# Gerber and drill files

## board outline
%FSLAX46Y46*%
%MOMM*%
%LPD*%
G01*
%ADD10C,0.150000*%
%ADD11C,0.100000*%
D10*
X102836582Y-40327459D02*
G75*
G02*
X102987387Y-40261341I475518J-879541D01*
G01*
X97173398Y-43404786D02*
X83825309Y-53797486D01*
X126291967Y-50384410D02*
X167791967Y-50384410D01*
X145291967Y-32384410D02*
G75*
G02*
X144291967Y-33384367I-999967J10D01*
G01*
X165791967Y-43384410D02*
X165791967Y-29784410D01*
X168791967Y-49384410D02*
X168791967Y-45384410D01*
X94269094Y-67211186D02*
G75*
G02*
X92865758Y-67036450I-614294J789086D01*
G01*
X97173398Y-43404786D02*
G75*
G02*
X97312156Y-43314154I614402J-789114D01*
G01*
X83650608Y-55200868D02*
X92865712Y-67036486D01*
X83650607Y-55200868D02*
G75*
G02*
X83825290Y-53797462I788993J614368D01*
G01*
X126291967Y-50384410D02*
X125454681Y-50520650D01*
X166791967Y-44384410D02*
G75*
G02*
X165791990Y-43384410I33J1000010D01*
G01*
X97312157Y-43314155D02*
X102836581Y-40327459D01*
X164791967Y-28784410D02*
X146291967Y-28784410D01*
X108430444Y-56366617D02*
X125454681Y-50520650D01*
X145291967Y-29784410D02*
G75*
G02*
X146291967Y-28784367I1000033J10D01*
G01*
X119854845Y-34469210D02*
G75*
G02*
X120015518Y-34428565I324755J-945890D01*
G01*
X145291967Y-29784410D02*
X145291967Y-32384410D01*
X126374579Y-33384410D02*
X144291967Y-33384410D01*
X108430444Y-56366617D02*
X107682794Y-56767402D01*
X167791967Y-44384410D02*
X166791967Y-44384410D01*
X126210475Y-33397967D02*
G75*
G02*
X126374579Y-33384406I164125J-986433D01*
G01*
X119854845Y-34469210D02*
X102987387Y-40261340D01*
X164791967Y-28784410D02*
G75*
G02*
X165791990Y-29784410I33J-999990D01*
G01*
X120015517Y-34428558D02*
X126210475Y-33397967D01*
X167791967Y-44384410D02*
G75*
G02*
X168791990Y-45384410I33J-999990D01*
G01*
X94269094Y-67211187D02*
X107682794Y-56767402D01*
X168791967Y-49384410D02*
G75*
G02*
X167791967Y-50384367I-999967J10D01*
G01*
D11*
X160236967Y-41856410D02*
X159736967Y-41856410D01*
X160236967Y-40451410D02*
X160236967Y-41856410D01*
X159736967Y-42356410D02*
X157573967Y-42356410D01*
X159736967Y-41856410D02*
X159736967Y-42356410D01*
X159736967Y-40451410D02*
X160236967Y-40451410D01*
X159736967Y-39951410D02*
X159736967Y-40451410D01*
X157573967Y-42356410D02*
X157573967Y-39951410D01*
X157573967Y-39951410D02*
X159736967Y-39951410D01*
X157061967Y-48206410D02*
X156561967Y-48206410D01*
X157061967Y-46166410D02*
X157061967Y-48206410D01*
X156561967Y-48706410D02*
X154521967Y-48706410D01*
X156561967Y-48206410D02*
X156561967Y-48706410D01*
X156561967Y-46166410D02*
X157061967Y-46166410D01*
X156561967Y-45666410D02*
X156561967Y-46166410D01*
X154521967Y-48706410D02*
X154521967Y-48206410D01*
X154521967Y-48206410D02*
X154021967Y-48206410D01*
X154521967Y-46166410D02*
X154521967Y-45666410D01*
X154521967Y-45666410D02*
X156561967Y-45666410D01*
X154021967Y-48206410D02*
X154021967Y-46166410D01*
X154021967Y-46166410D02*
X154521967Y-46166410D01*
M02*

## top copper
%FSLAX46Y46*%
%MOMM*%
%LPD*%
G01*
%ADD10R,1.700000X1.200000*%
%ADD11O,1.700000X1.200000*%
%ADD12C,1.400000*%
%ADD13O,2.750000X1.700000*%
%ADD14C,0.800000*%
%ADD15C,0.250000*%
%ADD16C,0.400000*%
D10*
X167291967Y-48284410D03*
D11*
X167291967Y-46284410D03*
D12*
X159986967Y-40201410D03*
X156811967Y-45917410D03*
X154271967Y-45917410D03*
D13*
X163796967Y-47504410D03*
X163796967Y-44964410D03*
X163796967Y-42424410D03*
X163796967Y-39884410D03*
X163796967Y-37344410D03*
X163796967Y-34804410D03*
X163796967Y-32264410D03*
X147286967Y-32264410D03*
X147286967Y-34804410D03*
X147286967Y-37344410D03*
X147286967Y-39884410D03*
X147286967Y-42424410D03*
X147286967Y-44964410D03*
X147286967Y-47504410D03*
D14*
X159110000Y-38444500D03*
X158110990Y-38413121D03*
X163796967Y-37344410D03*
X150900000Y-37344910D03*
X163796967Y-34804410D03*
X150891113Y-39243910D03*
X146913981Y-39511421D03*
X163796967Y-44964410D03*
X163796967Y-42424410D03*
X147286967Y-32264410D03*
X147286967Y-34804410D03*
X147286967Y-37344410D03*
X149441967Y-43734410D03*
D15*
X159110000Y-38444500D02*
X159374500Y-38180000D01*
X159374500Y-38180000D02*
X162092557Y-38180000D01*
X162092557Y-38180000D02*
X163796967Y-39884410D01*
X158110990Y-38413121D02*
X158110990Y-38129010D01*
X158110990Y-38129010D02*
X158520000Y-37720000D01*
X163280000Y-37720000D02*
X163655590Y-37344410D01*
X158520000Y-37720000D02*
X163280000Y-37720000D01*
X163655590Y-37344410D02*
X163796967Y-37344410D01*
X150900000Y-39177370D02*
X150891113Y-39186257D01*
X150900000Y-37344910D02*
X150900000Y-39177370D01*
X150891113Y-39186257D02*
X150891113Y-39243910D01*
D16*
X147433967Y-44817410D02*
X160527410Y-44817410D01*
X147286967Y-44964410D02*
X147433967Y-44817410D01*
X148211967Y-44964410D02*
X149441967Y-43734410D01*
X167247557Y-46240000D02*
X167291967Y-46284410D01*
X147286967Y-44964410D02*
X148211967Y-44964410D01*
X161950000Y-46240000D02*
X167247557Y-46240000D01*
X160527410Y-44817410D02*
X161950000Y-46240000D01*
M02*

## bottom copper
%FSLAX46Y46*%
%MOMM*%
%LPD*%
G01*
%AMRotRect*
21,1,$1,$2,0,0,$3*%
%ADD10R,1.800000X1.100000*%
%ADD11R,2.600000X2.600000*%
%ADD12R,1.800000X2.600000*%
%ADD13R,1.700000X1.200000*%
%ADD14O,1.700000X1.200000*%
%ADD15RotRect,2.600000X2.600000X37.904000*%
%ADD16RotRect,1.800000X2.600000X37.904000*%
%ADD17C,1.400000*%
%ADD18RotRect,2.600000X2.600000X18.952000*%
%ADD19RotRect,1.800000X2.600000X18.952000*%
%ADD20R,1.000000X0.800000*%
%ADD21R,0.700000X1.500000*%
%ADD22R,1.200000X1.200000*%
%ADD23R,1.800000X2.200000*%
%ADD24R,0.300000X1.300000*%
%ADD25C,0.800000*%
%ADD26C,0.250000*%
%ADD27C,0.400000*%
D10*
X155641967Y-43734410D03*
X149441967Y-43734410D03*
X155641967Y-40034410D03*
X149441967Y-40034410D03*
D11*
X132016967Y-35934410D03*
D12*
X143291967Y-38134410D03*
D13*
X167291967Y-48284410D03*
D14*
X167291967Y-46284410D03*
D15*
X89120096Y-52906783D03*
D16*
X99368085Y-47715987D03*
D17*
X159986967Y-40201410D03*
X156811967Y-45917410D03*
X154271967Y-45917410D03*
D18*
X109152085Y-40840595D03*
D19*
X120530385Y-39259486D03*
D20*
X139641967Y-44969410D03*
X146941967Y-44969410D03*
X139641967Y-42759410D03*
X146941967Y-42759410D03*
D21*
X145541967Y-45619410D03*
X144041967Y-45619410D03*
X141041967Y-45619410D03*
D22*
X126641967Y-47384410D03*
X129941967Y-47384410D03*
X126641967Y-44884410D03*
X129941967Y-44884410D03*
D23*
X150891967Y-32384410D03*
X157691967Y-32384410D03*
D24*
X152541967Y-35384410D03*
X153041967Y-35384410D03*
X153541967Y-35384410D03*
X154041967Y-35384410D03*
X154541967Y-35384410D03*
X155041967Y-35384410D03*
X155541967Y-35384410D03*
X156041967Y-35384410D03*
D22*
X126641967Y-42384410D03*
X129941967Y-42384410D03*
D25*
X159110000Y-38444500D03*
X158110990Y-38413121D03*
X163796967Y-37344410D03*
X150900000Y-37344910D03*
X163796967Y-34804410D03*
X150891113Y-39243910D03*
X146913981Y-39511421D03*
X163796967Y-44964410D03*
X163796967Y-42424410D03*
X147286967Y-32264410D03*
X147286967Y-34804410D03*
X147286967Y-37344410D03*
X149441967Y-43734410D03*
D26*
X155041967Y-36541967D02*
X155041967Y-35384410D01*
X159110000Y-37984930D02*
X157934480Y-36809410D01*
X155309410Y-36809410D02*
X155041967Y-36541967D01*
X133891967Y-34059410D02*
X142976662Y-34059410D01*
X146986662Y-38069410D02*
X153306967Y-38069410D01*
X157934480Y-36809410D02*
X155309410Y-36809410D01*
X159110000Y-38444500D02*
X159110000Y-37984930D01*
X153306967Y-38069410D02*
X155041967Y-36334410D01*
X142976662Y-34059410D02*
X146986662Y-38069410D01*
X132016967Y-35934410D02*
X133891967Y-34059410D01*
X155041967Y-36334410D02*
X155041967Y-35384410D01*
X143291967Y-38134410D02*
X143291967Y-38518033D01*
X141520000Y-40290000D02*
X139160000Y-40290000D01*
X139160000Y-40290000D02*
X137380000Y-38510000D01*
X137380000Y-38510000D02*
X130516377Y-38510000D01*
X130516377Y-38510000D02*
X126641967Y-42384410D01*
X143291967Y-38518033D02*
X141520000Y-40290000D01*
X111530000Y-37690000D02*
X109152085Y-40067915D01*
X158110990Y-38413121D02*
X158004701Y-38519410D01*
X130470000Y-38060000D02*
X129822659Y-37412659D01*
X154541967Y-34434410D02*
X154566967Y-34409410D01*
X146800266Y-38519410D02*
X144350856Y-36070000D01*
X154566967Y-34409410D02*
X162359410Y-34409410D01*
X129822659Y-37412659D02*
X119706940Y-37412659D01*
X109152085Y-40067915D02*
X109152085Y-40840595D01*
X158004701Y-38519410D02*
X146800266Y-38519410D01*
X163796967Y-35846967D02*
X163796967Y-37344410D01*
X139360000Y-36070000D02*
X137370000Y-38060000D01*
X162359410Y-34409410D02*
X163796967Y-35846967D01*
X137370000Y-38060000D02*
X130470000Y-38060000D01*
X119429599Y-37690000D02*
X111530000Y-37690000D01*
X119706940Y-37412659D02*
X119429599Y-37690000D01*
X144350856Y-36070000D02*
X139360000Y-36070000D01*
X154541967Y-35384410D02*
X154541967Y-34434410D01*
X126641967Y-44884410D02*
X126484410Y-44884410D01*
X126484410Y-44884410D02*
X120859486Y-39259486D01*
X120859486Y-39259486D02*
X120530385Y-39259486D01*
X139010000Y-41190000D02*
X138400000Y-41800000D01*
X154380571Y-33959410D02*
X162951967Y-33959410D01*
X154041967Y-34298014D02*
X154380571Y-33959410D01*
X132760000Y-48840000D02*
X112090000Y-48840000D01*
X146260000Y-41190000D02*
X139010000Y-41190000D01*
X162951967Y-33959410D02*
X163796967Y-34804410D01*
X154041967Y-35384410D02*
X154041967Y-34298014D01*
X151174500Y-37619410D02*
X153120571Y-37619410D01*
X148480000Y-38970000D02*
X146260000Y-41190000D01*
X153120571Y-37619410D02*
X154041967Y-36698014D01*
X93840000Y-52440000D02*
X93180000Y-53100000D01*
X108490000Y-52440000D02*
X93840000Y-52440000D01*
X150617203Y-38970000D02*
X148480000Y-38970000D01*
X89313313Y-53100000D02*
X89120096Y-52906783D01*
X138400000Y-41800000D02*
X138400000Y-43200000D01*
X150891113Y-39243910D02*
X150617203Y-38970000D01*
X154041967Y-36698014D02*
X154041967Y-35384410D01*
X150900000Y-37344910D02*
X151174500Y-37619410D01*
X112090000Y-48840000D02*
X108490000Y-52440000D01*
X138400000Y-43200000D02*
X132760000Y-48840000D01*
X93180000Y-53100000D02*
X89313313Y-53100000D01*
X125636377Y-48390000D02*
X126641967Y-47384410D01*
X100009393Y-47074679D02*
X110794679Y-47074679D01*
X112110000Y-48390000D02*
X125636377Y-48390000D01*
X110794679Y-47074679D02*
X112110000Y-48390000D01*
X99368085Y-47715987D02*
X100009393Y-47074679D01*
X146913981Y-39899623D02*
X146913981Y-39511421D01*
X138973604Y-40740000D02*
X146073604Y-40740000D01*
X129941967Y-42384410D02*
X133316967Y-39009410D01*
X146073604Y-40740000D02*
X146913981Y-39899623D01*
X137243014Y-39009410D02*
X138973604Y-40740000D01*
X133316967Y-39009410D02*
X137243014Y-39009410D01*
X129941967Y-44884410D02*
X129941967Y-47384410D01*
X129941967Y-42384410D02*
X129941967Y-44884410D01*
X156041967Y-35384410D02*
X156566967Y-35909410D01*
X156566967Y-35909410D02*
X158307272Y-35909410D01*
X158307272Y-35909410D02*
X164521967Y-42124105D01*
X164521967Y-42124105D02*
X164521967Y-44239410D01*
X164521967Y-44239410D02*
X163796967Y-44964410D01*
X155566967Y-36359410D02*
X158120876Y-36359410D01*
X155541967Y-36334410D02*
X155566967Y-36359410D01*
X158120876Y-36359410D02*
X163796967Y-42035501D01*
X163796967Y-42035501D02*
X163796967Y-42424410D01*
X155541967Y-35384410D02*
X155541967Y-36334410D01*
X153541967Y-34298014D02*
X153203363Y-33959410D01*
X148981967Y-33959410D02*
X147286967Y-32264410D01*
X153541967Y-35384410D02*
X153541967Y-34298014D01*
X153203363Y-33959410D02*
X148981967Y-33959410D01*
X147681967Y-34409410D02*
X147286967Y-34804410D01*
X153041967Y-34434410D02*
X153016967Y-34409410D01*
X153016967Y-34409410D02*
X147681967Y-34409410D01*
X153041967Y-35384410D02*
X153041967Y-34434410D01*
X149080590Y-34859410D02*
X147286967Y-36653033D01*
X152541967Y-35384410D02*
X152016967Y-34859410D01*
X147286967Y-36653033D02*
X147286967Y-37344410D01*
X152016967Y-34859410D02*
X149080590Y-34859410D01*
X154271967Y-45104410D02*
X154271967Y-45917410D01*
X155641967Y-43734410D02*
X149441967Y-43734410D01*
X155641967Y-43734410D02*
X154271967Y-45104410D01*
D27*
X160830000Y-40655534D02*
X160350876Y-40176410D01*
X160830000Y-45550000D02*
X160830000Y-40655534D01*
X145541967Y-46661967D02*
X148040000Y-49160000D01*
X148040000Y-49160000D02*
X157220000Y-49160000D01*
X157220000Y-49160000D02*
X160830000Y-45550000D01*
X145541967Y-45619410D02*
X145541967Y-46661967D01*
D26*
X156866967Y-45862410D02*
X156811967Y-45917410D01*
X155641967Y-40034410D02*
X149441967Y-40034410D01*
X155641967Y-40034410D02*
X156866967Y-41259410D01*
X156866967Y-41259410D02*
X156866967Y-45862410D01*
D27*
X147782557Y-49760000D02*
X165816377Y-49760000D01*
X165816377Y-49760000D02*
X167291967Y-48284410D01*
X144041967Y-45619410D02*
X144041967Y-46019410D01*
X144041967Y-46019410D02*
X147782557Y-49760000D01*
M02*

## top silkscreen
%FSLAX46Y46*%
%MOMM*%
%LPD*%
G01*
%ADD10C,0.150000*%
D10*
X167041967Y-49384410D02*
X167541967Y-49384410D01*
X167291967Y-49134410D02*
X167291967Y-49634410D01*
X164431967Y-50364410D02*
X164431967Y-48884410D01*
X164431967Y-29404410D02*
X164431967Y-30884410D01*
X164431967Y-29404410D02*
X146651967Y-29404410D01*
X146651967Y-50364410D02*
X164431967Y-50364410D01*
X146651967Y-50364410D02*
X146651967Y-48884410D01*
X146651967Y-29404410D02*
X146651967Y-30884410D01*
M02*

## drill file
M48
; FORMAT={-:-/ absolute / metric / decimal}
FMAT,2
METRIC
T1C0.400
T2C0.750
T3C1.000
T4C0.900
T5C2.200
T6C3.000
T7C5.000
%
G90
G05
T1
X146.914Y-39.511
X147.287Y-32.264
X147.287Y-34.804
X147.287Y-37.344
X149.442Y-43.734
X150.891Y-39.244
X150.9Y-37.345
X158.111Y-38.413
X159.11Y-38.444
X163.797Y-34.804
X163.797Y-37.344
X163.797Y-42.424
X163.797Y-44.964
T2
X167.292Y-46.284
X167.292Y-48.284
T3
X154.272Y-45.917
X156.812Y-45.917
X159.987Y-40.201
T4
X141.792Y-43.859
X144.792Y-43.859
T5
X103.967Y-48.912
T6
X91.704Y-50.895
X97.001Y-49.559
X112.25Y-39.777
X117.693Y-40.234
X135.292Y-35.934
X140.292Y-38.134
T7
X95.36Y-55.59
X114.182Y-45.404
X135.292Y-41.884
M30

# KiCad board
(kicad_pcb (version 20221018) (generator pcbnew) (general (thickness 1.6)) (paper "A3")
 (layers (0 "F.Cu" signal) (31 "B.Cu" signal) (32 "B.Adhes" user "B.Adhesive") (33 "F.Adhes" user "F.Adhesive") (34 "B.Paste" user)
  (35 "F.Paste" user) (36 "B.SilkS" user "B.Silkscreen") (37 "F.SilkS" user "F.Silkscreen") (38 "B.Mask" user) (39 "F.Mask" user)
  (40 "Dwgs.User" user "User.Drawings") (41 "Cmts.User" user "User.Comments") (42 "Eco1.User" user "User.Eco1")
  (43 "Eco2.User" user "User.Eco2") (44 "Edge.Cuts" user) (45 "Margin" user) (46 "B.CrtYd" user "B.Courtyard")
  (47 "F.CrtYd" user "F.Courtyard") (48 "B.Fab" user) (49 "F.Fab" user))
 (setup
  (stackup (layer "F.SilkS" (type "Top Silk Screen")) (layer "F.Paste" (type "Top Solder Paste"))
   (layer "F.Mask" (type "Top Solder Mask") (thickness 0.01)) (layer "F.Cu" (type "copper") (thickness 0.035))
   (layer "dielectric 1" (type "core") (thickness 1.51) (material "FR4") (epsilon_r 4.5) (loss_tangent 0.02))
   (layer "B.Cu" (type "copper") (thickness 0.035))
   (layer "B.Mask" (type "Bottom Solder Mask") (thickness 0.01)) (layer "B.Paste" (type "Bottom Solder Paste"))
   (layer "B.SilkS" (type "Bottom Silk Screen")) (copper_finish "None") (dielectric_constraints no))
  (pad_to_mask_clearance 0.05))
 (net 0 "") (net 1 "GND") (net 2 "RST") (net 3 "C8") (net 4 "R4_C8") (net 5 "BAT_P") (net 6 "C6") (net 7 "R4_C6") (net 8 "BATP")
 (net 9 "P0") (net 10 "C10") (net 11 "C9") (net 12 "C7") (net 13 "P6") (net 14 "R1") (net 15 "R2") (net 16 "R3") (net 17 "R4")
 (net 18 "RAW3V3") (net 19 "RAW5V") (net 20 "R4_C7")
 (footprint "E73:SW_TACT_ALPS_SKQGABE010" (layer "F.Cu") (at 152.541967 41.88441 180)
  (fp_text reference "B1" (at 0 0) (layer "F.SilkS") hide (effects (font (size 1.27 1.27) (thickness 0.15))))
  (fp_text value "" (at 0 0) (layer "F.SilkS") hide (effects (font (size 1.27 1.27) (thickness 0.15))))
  (pad "1" smd rect (at -3.1 -1.85 180) (size 1.8 1.1) (layers "B.Cu" "B.Paste" "B.Mask") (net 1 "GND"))
  (pad "1" smd rect (at 3.1 -1.85 180) (size 1.8 1.1) (layers "B.Cu" "B.Paste" "B.Mask") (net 1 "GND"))
  (pad "2" smd rect (at -3.1 1.85 180) (size 1.8 1.1) (layers "B.Cu" "B.Paste" "B.Mask") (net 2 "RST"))
  (pad "2" smd rect (at 3.1 1.85 180) (size 1.8 1.1) (layers "B.Cu" "B.Paste" "B.Mask") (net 2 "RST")))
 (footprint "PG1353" (layer "F.Cu") (at 135.291967 41.88441)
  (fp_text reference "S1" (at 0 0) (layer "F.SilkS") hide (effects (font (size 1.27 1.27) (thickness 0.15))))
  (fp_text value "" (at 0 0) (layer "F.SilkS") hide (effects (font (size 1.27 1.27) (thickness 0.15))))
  (pad "" np_thru_hole circle (at 0 -5.95) (size 3 3) (drill 3) (layers "*.Cu" "*.Mask"))
  (pad "" np_thru_hole circle (at 0 0) (size 5 5) (drill 5) (layers "*.Cu" "*.Mask"))
  (pad "" np_thru_hole circle (at 5 -3.75) (size 3 3) (drill 3) (layers "*.Cu" "*.Mask"))
  (pad "1" smd rect (at -3.275 -5.95) (size 2.6 2.6) (layers "B.Cu" "B.Paste" "B.Mask") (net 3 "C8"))
  (pad "2" smd rect (at 8 -3.75) (size 1.8 2.6) (layers "B.Cu" "B.Paste" "B.Mask") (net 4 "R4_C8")))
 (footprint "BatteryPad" (layer "F.Cu") (at 167.291967 47.28441 90)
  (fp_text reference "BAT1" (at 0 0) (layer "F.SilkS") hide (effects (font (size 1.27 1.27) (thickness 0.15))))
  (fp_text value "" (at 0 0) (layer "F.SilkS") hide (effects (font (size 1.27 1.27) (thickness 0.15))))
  (fp_line (start -2.1 -0.25) (end -2.1 0.25) (stroke (width 0.15) (type solid)) (layer "F.SilkS"))
  (fp_line (start -1.85 0) (end -2.35 0) (stroke (width 0.15) (type solid)) (layer "F.SilkS"))
  (pad "1" thru_hole rect (at -1 0 90) (size 1.2 1.7) (drill 0.75) (layers "*.Cu" "*.Mask") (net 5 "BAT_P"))
  (pad "2" thru_hole oval (at 1 0 90) (size 1.2 1.7) (drill 0.75) (layers "*.Cu" "*.Mask") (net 1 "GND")))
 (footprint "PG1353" (layer "F.Cu") (at 95.359531 55.589614 37.904)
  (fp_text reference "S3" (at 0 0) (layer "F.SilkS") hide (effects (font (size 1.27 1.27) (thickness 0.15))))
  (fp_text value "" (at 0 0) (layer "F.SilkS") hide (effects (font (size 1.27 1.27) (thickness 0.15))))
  (pad "" np_thru_hole circle (at 0 -5.95) (size 3 3) (drill 3) (layers "*.Cu" "*.Mask"))
  (pad "" np_thru_hole circle (at 0 0) (size 5 5) (drill 5) (layers "*.Cu" "*.Mask"))
  (pad "" np_thru_hole circle (at 5 -3.75) (size 3 3) (drill 3) (layers "*.Cu" "*.Mask"))
  (pad "1" smd rect (at -3.275 -5.95 37.904) (size 2.6 2.6) (layers "B.Cu" "B.Paste" "B.Mask") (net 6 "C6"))
  (pad "2" smd rect (at 8 -3.75 37.904) (size 1.8 2.6) (layers "B.Cu" "B.Paste" "B.Mask") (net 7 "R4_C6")))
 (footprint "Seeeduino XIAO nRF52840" (layer "F.Cu") (at 155.541967 39.88441 180)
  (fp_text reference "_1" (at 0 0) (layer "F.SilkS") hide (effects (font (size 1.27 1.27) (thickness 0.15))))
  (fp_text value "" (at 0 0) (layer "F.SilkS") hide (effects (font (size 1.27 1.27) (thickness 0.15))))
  (fp_line (start -8.89 -10.48) (end -8.89 -9) (stroke (width 0.15) (type solid)) (layer "F.SilkS"))
  (fp_line (start -8.89 10.48) (end -8.89 9) (stroke (width 0.15) (type solid)) (layer "F.SilkS"))
  (fp_line (start -8.89 10.48) (end 8.89 10.48) (stroke (width 0.15) (type solid)) (layer "F.SilkS"))
  (fp_line (start 8.89 -10.48) (end -8.89 -10.48) (stroke (width 0.15) (type solid)) (layer "F.SilkS"))
  (fp_line (start 8.89 -10.48) (end 8.89 -9) (stroke (width 0.15) (type solid)) (layer "F.SilkS"))
  (fp_line (start 8.89 10.48) (end 8.89 9) (stroke (width 0.15) (type solid)) (layer "F.SilkS"))
  (fp_line (start -4.695 -1.972) (end -4.195 -1.972) (stroke (width 0.1) (type solid)) (layer "Edge.Cuts"))
  (fp_line (start -4.695 -0.567) (end -4.695 -1.972) (stroke (width 0.1) (type solid)) (layer "Edge.Cuts"))
  (fp_line (start -4.195 -2.472) (end -2.032 -2.472) (stroke (width 0.1) (type solid)) (layer "Edge.Cuts"))
  (fp_line (start -4.195 -1.972) (end -4.195 -2.472) (stroke (width 0.1) (type solid)) (layer "Edge.Cuts"))
  (fp_line (start -4.195 -0.567) (end -4.695 -0.567) (stroke (width 0.1) (type solid)) (layer "Edge.Cuts"))
  (fp_line (start -4.195 -0.067) (end -4.195 -0.567) (stroke (width 0.1) (type solid)) (layer "Edge.Cuts"))
  (fp_line (start -2.032 -2.472) (end -2.032 -0.067) (stroke (width 0.1) (type solid)) (layer "Edge.Cuts"))
  (fp_line (start -2.032 -0.067) (end -4.195 -0.067) (stroke (width 0.1) (type solid)) (layer "Edge.Cuts"))
  (fp_line (start -1.52 -8.322) (end -1.02 -8.322) (stroke (width 0.1) (type solid)) (layer "Edge.Cuts"))
  (fp_line (start -1.52 -6.282) (end -1.52 -8.322) (stroke (width 0.1) (type solid)) (layer "Edge.Cuts"))
  (fp_line (start -1.02 -8.822) (end 1.02 -8.822) (stroke (width 0.1) (type solid)) (layer "Edge.Cuts"))
  (fp_line (start -1.02 -8.322) (end -1.02 -8.822) (stroke (width 0.1) (type solid)) (layer "Edge.Cuts"))
  (fp_line (start -1.02 -6.282) (end -1.52 -6.282) (stroke (width 0.1) (type solid)) (layer "Edge.Cuts"))
  (fp_line (start -1.02 -5.782) (end -1.02 -6.282) (stroke (width 0.1) (type solid)) (layer "Edge.Cuts"))
  (fp_line (start 1.02 -8.822) (end 1.02 -8.322) (stroke (width 0.1) (type solid)) (layer "Edge.Cuts"))
  (fp_line (start 1.02 -8.322) (end 1.52 -8.322) (stroke (width 0.1) (type solid)) (layer "Edge.Cuts"))
  (fp_line (start 1.02 -6.282) (end 1.02 -5.782) (stroke (width 0.1) (type solid)) (layer "Edge.Cuts"))
  (fp_line (start 1.02 -5.782) (end -1.02 -5.782) (stroke (width 0.1) (type solid)) (layer "Edge.Cuts"))
  (fp_line (start 1.52 -8.322) (end 1.52 -6.282) (stroke (width 0.1) (type solid)) (layer "Edge.Cuts"))
  (fp_line (start 1.52 -6.282) (end 1.02 -6.282) (stroke (width 0.1) (type solid)) (layer "Edge.Cuts"))
  (pad "" thru_hole circle (at -4.445 -0.317) (size 1.4 1.4) (drill 1) (layers "*.Cu" "*.Mask") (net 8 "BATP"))
  (pad "" thru_hole circle (at -1.27 -6.033) (size 1.4 1.4) (drill 1) (layers "*.Cu" "*.Mask") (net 2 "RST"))
  (pad "" thru_hole circle (at 1.27 -6.033) (size 1.4 1.4) (drill 1) (layers "*.Cu" "*.Mask") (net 1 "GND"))
  (pad "1" smd oval (at -8.255 -7.62 180) (size 2.75 1.7) (layers "F.Cu" "F.Paste" "F.Mask") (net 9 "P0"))
  (pad "2" smd oval (at -8.255 -5.08 180) (size 2.75 1.7) (layers "F.Cu" "F.Paste" "F.Mask") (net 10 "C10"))
  (pad "3" smd oval (at -8.255 -2.54 180) (size 2.75 1.7) (layers "F.Cu" "F.Paste" "F.Mask") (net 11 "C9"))
  (pad "4" smd oval (at -8.255 0 180) (size 2.75 1.7) (layers "F.Cu" "F.Paste" "F.Mask") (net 3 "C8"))
  (pad "5" smd oval (at -8.255 2.54 180) (size 2.75 1.7) (layers "F.Cu" "F.Paste" "F.Mask") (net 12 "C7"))
  (pad "6" smd oval (at -8.255 5.08 180) (size 2.75 1.7) (layers "F.Cu" "F.Paste" "F.Mask") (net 6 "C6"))
  (pad "7" smd oval (at -8.255 7.62 180) (size 2.75 1.7) (layers "F.Cu" "F.Paste" "F.Mask") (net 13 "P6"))
  (pad "8" smd oval (at 8.255 7.62 180) (size 2.75 1.7) (layers "F.Cu" "F.Paste" "F.Mask") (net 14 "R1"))
  (pad "9" smd oval (at 8.255 5.08 180) (size 2.75 1.7) (layers "F.Cu" "F.Paste" "F.Mask") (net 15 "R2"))
  (pad "10" smd oval (at 8.255 2.54 180) (size 2.75 1.7) (layers "F.Cu" "F.Paste" "F.Mask") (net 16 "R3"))
  (pad "11" smd oval (at 8.255 0 180) (size 2.75 1.7) (layers "F.Cu" "F.Paste" "F.Mask") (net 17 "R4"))
  (pad "12" smd oval (at 8.255 -2.54 180) (size 2.75 1.7) (layers "F.Cu" "F.Paste" "F.Mask") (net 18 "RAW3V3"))
  (pad "13" smd oval (at 8.255 -5.08 180) (size 2.75 1.7) (layers "F.Cu" "F.Paste" "F.Mask") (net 1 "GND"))
  (pad "14" smd oval (at 8.255 -7.62 180) (size 2.75 1.7) (layers "F.Cu" "F.Paste" "F.Mask") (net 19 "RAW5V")))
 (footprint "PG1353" (layer "F.Cu") (at 114.181967 45.40441 18.952)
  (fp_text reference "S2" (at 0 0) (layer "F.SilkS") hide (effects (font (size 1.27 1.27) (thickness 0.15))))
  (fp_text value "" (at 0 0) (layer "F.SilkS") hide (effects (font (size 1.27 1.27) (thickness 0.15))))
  (pad "" np_thru_hole circle (at 0 -5.95) (size 3 3) (drill 3) (layers "*.Cu" "*.Mask"))
  (pad "" np_thru_hole circle (at 0 0) (size 5 5) (drill 5) (layers "*.Cu" "*.Mask"))
  (pad "" np_thru_hole circle (at 5 -3.75) (size 3 3) (drill 3) (layers "*.Cu" "*.Mask"))
  (pad "1" smd rect (at -3.275 -5.95 18.952) (size 2.6 2.6) (layers "B.Cu" "B.Paste" "B.Mask") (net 12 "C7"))
  (pad "2" smd rect (at 8 -3.75 18.952) (size 1.8 2.6) (layers "B.Cu" "B.Paste" "B.Mask") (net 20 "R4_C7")))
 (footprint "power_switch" (layer "F.Cu") (at 143.291967 43.88441 90)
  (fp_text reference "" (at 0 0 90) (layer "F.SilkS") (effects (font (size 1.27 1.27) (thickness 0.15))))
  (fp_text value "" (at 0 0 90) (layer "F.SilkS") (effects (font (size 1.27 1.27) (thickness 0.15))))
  (pad "" smd rect (at -1.085 -3.65) (size 1 0.8) (layers "B.Cu" "B.Paste" "B.Mask"))
  (pad "" smd rect (at -1.085 3.65) (size 1 0.8) (layers "B.Cu" "B.Paste" "B.Mask"))
  (pad "" np_thru_hole circle (at 0.025 -1.5 180) (size 0.9 0.9) (drill 0.9) (layers "*.Cu" "*.Mask"))
  (pad "" np_thru_hole circle (at 0.025 1.5 180) (size 0.9 0.9) (drill 0.9) (layers "*.Cu" "*.Mask"))
  (pad "" smd rect (at 1.125 -3.65) (size 1 0.8) (layers "B.Cu" "B.Paste" "B.Mask"))
  (pad "" smd rect (at 1.125 3.65) (size 1 0.8) (layers "B.Cu" "B.Paste" "B.Mask"))
  (pad "4" smd rect (at -1.735 2.25) (size 0.7 1.5) (layers "B.Cu" "B.Paste" "B.Mask") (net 8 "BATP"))
  (pad "5" smd rect (at -1.735 0.75) (size 0.7 1.5) (layers "B.Cu" "B.Paste" "B.Mask") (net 5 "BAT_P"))
  (pad "6" smd rect (at -1.735 -2.25) (size 0.7 1.5) (layers "B.Cu" "B.Paste" "B.Mask")))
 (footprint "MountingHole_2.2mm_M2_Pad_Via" (layer "F.Cu") (at 103.967424 48.91199 18.952)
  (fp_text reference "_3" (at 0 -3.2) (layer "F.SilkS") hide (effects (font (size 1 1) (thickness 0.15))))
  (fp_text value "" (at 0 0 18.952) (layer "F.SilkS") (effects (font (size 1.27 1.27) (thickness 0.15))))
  (pad "" np_thru_hole circle (at 0 0) (size 2.2 2.2) (drill 2.2) (layers "*.Cu" "*.Mask")))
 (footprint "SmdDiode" (layer "B.Cu") (at 128.291967 44.88441 90)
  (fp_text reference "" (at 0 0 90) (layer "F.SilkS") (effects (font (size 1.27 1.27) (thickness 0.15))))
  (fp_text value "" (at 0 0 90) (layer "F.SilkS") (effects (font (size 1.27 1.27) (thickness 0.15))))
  (pad "1" smd rect (at -2.5 -1.65 90) (size 1.2 1.2) (layers "B.Cu" "B.Paste" "B.Mask") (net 7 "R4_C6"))
  (pad "2" smd rect (at -2.5 1.65 90) (size 1.2 1.2) (layers "B.Cu" "B.Paste" "B.Mask") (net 17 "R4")))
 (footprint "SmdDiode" (layer "B.Cu") (at 128.291967 44.88441 90)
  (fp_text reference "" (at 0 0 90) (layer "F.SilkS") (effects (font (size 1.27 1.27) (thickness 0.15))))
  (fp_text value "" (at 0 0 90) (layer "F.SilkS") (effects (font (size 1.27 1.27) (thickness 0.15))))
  (pad "1" smd rect (at 0 -1.65 90) (size 1.2 1.2) (layers "B.Cu" "B.Paste" "B.Mask") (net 20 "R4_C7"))
  (pad "2" smd rect (at 0 1.65 90) (size 1.2 1.2) (layers "B.Cu" "B.Paste" "B.Mask") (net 17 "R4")))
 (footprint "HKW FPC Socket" (layer "B.Cu") (at 154.291967 32.38441)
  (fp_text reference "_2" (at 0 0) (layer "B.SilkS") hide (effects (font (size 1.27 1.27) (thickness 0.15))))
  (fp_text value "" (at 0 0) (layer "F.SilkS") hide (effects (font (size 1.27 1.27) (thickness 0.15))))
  (pad "" smd rect (at -3.4 0) (size 1.8 2.2) (layers "B.Cu" "B.Paste" "B.Mask"))
  (pad "" smd rect (at 3.4 0) (size 1.8 2.2) (layers "B.Cu" "B.Paste" "B.Mask"))
  (pad "1" smd rect (at -1.75 3) (size 0.3 1.3) (layers "B.Cu" "B.Paste" "B.Mask") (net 16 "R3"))
  (pad "2" smd rect (at -1.25 3) (size 0.3 1.3) (layers "B.Cu" "B.Paste" "B.Mask") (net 15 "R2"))
  (pad "3" smd rect (at -0.75 3) (size 0.3 1.3) (layers "B.Cu" "B.Paste" "B.Mask") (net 14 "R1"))
  (pad "4" smd rect (at -0.25 3) (size 0.3 1.3) (layers "B.Cu" "B.Paste" "B.Mask") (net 6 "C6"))
  (pad "5" smd rect (at 0.25 3) (size 0.3 1.3) (layers "B.Cu" "B.Paste" "B.Mask") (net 12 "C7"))
  (pad "6" smd rect (at 0.75 3) (size 0.3 1.3) (layers "B.Cu" "B.Paste" "B.Mask") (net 3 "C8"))
  (pad "7" smd rect (at 1.25 3) (size 0.3 1.3) (layers "B.Cu" "B.Paste" "B.Mask") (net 11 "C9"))
  (pad "8" smd rect (at 1.75 3) (size 0.3 1.3) (layers "B.Cu" "B.Paste" "B.Mask") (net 10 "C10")))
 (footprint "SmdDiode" (layer "B.Cu") (at 128.291967 44.88441 90)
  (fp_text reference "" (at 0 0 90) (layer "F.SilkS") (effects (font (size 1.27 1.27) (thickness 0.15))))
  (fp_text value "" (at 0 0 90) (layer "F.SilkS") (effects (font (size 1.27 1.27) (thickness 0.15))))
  (pad "1" smd rect (at 2.5 -1.65 90) (size 1.2 1.2) (layers "B.Cu" "B.Paste" "B.Mask") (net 4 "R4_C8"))
  (pad "2" smd rect (at 2.5 1.65 90) (size 1.2 1.2) (layers "B.Cu" "B.Paste" "B.Mask") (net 17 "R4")))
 (gr_arc (start 102.836582 40.327459) (mid 102.910621 40.29129) (end 102.987387 40.26134) (stroke (width 0.15) (type solid))
  (layer "Edge.Cuts"))
 (gr_line (start 97.173398 43.404786) (end 83.825309 53.797486) (stroke (width 0.15) (type solid)) (layer "Edge.Cuts"))
 (gr_line (start 126.291967 50.38441) (end 167.791967 50.38441) (stroke (width 0.15) (type solid)) (layer "Edge.Cuts"))
 (gr_arc (start 145.291967 32.38441) (mid 144.999074 33.091517) (end 144.291967 33.38441) (stroke (width 0.15) (type solid))
  (layer "Edge.Cuts"))
 (gr_line (start 165.791967 43.38441) (end 165.791967 29.78441) (stroke (width 0.15) (type solid)) (layer "Edge.Cuts"))
 (gr_line (start 168.791967 49.38441) (end 168.791967 45.38441) (stroke (width 0.15) (type solid)) (layer "Edge.Cuts"))
 (gr_arc (start 94.269094 67.211186) (mid 93.531221 67.414486) (end 92.865712 67.036486) (stroke (width 0.15) (type solid))
  (layer "Edge.Cuts"))
 (gr_arc (start 97.173398 43.404786) (mid 97.240897 43.356591) (end 97.312157 43.314155) (stroke (width 0.15) (type solid))
  (layer "Edge.Cuts"))
 (gr_line (start 83.650608 55.200868) (end 92.865712 67.036486) (stroke (width 0.15) (type solid)) (layer "Edge.Cuts"))
 (gr_arc (start 83.650607 55.200868) (mid 83.447308 54.462995) (end 83.825309 53.797486) (stroke (width 0.15) (type solid))
  (layer "Edge.Cuts"))
 (gr_line (start 126.291967 50.38441) (end 125.454681 50.52065) (stroke (width 0.15) (type solid)) (layer "Edge.Cuts"))
 (gr_arc (start 166.791967 44.38441) (mid 166.08486 44.091517) (end 165.791967 43.38441) (stroke (width 0.15) (type solid))
  (layer "Edge.Cuts"))
 (gr_line (start 97.312157 43.314155) (end 102.836581 40.327459) (stroke (width 0.15) (type solid)) (layer "Edge.Cuts"))
 (gr_line (start 164.791967 28.78441) (end 146.291967 28.78441) (stroke (width 0.15) (type solid)) (layer "Edge.Cuts"))
 (gr_line (start 108.430444 56.366617) (end 125.454681 50.52065) (stroke (width 0.15) (type solid)) (layer "Edge.Cuts"))
 (gr_arc (start 145.291967 29.78441) (mid 145.58486 29.077303) (end 146.291967 28.78441) (stroke (width 0.15) (type solid))
  (layer "Edge.Cuts"))
 (gr_arc (start 119.854845 34.46921) (mid 119.934337 34.44555) (end 120.015517 34.428558) (stroke (width 0.15) (type solid))
  (layer "Edge.Cuts"))
 (gr_line (start 145.291967 29.78441) (end 145.291967 32.38441) (stroke (width 0.15) (type solid)) (layer "Edge.Cuts"))
 (gr_line (start 126.374579 33.38441) (end 144.291967 33.38441) (stroke (width 0.15) (type solid)) (layer "Edge.Cuts"))
 (gr_line (start 108.430444 56.366617) (end 107.682794 56.767402) (stroke (width 0.15) (type solid)) (layer "Edge.Cuts"))
 (gr_line (start 167.791967 44.38441) (end 166.791967 44.38441) (stroke (width 0.15) (type solid)) (layer "Edge.Cuts"))
 (gr_arc (start 126.210475 33.397967) (mid 126.292247 33.387805) (end 126.374579 33.38441) (stroke (width 0.15) (type solid))
  (layer "Edge.Cuts"))
 (gr_line (start 119.854845 34.46921) (end 102.987387 40.26134) (stroke (width 0.15) (type solid)) (layer "Edge.Cuts"))
 (gr_arc (start 164.791967 28.78441) (mid 165.499074 29.077303) (end 165.791967 29.78441) (stroke (width 0.15) (type solid))
  (layer "Edge.Cuts"))
 (gr_line (start 120.015517 34.428558) (end 126.210475 33.397967) (stroke (width 0.15) (type solid)) (layer "Edge.Cuts"))
 (gr_arc (start 167.791967 44.38441) (mid 168.499074 44.677303) (end 168.791967 45.38441) (stroke (width 0.15) (type solid))
  (layer "Edge.Cuts"))
 (gr_line (start 94.269094 67.211187) (end 107.682794 56.767402) (stroke (width 0.15) (type solid)) (layer "Edge.Cuts"))
 (gr_arc (start 168.791967 49.38441) (mid 168.499074 50.091517) (end 167.791967 50.38441) (stroke (width 0.15) (type solid))
  (layer "Edge.Cuts"))
 (segment (start 159.11 38.4445) (end 159.3745 38.18) (width 0.25) (layer "F.Cu") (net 3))
 (segment (start 159.3745 38.18) (end 162.092557 38.18) (width 0.25) (layer "F.Cu") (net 3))
 (segment (start 162.092557 38.18) (end 163.796967 39.88441) (width 0.25) (layer "F.Cu") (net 3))
 (via (at 159.11 38.4445) (size 0.8) (drill 0.4) (layers "F.Cu" "B.Cu") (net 3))
 (segment (start 155.041967 36.541967) (end 155.041967 35.38441) (width 0.25) (layer "B.Cu") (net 3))
 (segment (start 159.11 37.98493) (end 157.93448 36.80941) (width 0.25) (layer "B.Cu") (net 3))
 (segment (start 155.30941 36.80941) (end 155.041967 36.541967) (width 0.25) (layer "B.Cu") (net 3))
 (segment (start 133.891967 34.05941) (end 142.976662 34.05941) (width 0.25) (layer "B.Cu") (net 3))
 (segment (start 146.986662 38.06941) (end 153.306967 38.06941) (width 0.25) (layer "B.Cu") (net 3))
 (segment (start 157.93448 36.80941) (end 155.30941 36.80941) (width 0.25) (layer "B.Cu") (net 3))
 (segment (start 159.11 38.4445) (end 159.11 37.98493) (width 0.25) (layer "B.Cu") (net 3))
 (segment (start 153.306967 38.06941) (end 155.041967 36.33441) (width 0.25) (layer "B.Cu") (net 3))
 (segment (start 142.976662 34.05941) (end 146.986662 38.06941) (width 0.25) (layer "B.Cu") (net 3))
 (segment (start 132.016967 35.93441) (end 133.891967 34.05941) (width 0.25) (layer "B.Cu") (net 3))
 (segment (start 155.041967 36.33441) (end 155.041967 35.38441) (width 0.25) (layer "B.Cu") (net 3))
 (segment (start 143.291967 38.13441) (end 143.291967 38.518033) (width 0.25) (layer "B.Cu") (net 4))
 (segment (start 141.52 40.29) (end 139.16 40.29) (width 0.25) (layer "B.Cu") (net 4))
 (segment (start 139.16 40.29) (end 137.38 38.51) (width 0.25) (layer "B.Cu") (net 4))
 (segment (start 137.38 38.51) (end 130.516377 38.51) (width 0.25) (layer "B.Cu") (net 4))
 (segment (start 130.516377 38.51) (end 126.641967 42.38441) (width 0.25) (layer "B.Cu") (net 4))
 (segment (start 143.291967 38.518033) (end 141.52 40.29) (width 0.25) (layer "B.Cu") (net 4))
 (segment (start 158.11099 38.413121) (end 158.11099 38.12901) (width 0.25) (layer "F.Cu") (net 12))
 (segment (start 158.11099 38.12901) (end 158.52 37.72) (width 0.25) (layer "F.Cu") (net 12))
 (segment (start 163.28 37.72) (end 163.65559 37.34441) (width 0.25) (layer "F.Cu") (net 12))
 (segment (start 158.52 37.72) (end 163.28 37.72) (width 0.25) (layer "F.Cu") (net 12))
 (segment (start 163.65559 37.34441) (end 163.796967 37.34441) (width 0.25) (layer "F.Cu") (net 12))
 (via (at 158.11099 38.413121) (size 0.8) (drill 0.4) (layers "F.Cu" "B.Cu") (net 12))
 (via (at 163.796967 37.34441) (size 0.8) (drill 0.4) (layers "F.Cu" "B.Cu") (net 12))
 (segment (start 111.53 37.69) (end 109.152085 40.067915) (width 0.25) (layer "B.Cu") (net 12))
 (segment (start 158.11099 38.413121) (end 158.004701 38.51941) (width 0.25) (layer "B.Cu") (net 12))
 (segment (start 130.47 38.06) (end 129.822659 37.412659) (width 0.25) (layer "B.Cu") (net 12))
 (segment (start 154.541967 34.43441) (end 154.566967 34.40941) (width 0.25) (layer "B.Cu") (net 12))
 (segment (start 146.800266 38.51941) (end 144.350856 36.07) (width 0.25) (layer "B.Cu") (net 12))
 (segment (start 154.566967 34.40941) (end 162.35941 34.40941) (width 0.25) (layer "B.Cu") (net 12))
 (segment (start 129.822659 37.412659) (end 119.70694 37.412659) (width 0.25) (layer "B.Cu") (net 12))
 (segment (start 109.152085 40.067915) (end 109.152085 40.840595) (width 0.25) (layer "B.Cu") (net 12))
 (segment (start 158.004701 38.51941) (end 146.800266 38.51941) (width 0.25) (layer "B.Cu") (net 12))
 (segment (start 163.796967 35.846967) (end 163.796967 37.34441) (width 0.25) (layer "B.Cu") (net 12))
 (segment (start 139.36 36.07) (end 137.37 38.06) (width 0.25) (layer "B.Cu") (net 12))
 (segment (start 162.35941 34.40941) (end 163.796967 35.846967) (width 0.25) (layer "B.Cu") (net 12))
 (segment (start 137.37 38.06) (end 130.47 38.06) (width 0.25) (layer "B.Cu") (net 12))
 (segment (start 119.429599 37.69) (end 111.53 37.69) (width 0.25) (layer "B.Cu") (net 12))
 (segment (start 119.70694 37.412659) (end 119.429599 37.69) (width 0.25) (layer "B.Cu") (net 12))
 (segment (start 144.350856 36.07) (end 139.36 36.07) (width 0.25) (layer "B.Cu") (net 12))
 (segment (start 154.541967 35.38441) (end 154.541967 34.43441) (width 0.25) (layer "B.Cu") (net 12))
 (segment (start 126.641967 44.88441) (end 126.48441 44.88441) (width 0.25) (layer "B.Cu") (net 20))
 (segment (start 126.48441 44.88441) (end 120.859486 39.259486) (width 0.25) (layer "B.Cu") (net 20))
 (segment (start 120.859486 39.259486) (end 120.530385 39.259486) (width 0.25) (layer "B.Cu") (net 20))
 (segment (start 150.9 39.17737) (end 150.891113 39.186257) (width 0.25) (layer "F.Cu") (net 6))
 (segment (start 150.9 37.34491) (end 150.9 39.17737) (width 0.25) (layer "F.Cu") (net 6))
 (segment (start 150.891113 39.186257) (end 150.891113 39.24391) (width 0.25) (layer "F.Cu") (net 6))
 (via (at 150.9 37.34491) (size 0.8) (drill 0.4) (layers "F.Cu" "B.Cu") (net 6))
 (via (at 163.796967 34.80441) (size 0.8) (drill 0.4) (layers "F.Cu" "B.Cu") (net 6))
 (via (at 150.891113 39.24391) (size 0.8) (drill 0.4) (layers "F.Cu" "B.Cu") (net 6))
 (segment (start 139.01 41.19) (end 138.4 41.8) (width 0.25) (layer "B.Cu") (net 6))
 (segment (start 154.380571 33.95941) (end 162.951967 33.95941) (width 0.25) (layer "B.Cu") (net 6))
 (segment (start 154.041967 34.298014) (end 154.380571 33.95941) (width 0.25) (layer "B.Cu") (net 6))
 (segment (start 132.76 48.84) (end 112.09 48.84) (width 0.25) (layer "B.Cu") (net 6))
 (segment (start 146.26 41.19) (end 139.01 41.19) (width 0.25) (layer "B.Cu") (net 6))
 (segment (start 162.951967 33.95941) (end 163.796967 34.80441) (width 0.25) (layer "B.Cu") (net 6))
 (segment (start 154.041967 35.38441) (end 154.041967 34.298014) (width 0.25) (layer "B.Cu") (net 6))
 (segment (start 151.1745 37.61941) (end 153.120571 37.61941) (width 0.25) (layer "B.Cu") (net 6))
 (segment (start 148.48 38.97) (end 146.26 41.19) (width 0.25) (layer "B.Cu") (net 6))
 (segment (start 153.120571 37.61941) (end 154.041967 36.698014) (width 0.25) (layer "B.Cu") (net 6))
 (segment (start 93.84 52.44) (end 93.18 53.1) (width 0.25) (layer "B.Cu") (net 6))
 (segment (start 108.49 52.44) (end 93.84 52.44) (width 0.25) (layer "B.Cu") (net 6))
 (segment (start 150.617203 38.97) (end 148.48 38.97) (width 0.25) (layer "B.Cu") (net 6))
 (segment (start 89.313313 53.1) (end 89.120096 52.906783) (width 0.25) (layer "B.Cu") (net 6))
 (segment (start 138.4 41.8) (end 138.4 43.2) (width 0.25) (layer "B.Cu") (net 6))
 (segment (start 150.891113 39.24391) (end 150.617203 38.97) (width 0.25) (layer "B.Cu") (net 6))
 (segment (start 154.041967 36.698014) (end 154.041967 35.38441) (width 0.25) (layer "B.Cu") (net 6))
 (segment (start 150.9 37.34491) (end 151.1745 37.61941) (width 0.25) (layer "B.Cu") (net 6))
 (segment (start 112.09 48.84) (end 108.49 52.44) (width 0.25) (layer "B.Cu") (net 6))
 (segment (start 138.4 43.2) (end 132.76 48.84) (width 0.25) (layer "B.Cu") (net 6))
 (segment (start 93.18 53.1) (end 89.313313 53.1) (width 0.25) (layer "B.Cu") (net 6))
 (segment (start 125.636377 48.39) (end 126.641967 47.38441) (width 0.25) (layer "B.Cu") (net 7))
 (segment (start 100.009393 47.074679) (end 110.794679 47.074679) (width 0.25) (layer "B.Cu") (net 7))
 (segment (start 112.11 48.39) (end 125.636377 48.39) (width 0.25) (layer "B.Cu") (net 7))
 (segment (start 110.794679 47.074679) (end 112.11 48.39) (width 0.25) (layer "B.Cu") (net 7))
 (segment (start 99.368085 47.715987) (end 100.009393 47.074679) (width 0.25) (layer "B.Cu") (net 7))
 (via (at 146.913981 39.511421) (size 0.8) (drill 0.4) (layers "F.Cu" "B.Cu") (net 17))
 (segment (start 146.913981 39.899623) (end 146.913981 39.511421) (width 0.25) (layer "B.Cu") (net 17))
 (segment (start 138.973604 40.74) (end 146.073604 40.74) (width 0.25) (layer "B.Cu") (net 17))
 (segment (start 129.941967 42.38441) (end 133.316967 39.00941) (width 0.25) (layer "B.Cu") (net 17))
 (segment (start 146.073604 40.74) (end 146.913981 39.899623) (width 0.25) (layer "B.Cu") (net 17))
 (segment (start 137.243014 39.00941) (end 138.973604 40.74) (width 0.25) (layer "B.Cu") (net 17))
 (segment (start 133.316967 39.00941) (end 137.243014 39.00941) (width 0.25) (layer "B.Cu") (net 17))
 (segment (start 129.941967 44.88441) (end 129.941967 47.38441) (width 0.25) (layer "B.Cu") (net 17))
 (segment (start 129.941967 42.38441) (end 129.941967 44.88441) (width 0.25) (layer "B.Cu") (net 17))
 (via (at 163.796967 44.96441) (size 0.8) (drill 0.4) (layers "F.Cu" "B.Cu") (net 10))
 (segment (start 156.041967 35.38441) (end 156.566967 35.90941) (width 0.25) (layer "B.Cu") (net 10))
 (segment (start 156.566967 35.90941) (end 158.307272 35.90941) (width 0.25) (layer "B.Cu") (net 10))
 (segment (start 158.307272 35.90941) (end 164.521967 42.124105) (width 0.25) (layer "B.Cu") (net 10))
 (segment (start 164.521967 42.124105) (end 164.521967 44.23941) (width 0.25) (layer "B.Cu") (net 10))
 (segment (start 164.521967 44.23941) (end 163.796967 44.96441) (width 0.25) (layer "B.Cu") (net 10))
 (via (at 163.796967 42.42441) (size 0.8) (drill 0.4) (layers "F.Cu" "B.Cu") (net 11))
 (segment (start 155.566967 36.35941) (end 158.120876 36.35941) (width 0.25) (layer "B.Cu") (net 11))
 (segment (start 155.541967 36.33441) (end 155.566967 36.35941) (width 0.25) (layer "B.Cu") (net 11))
 (segment (start 158.120876 36.35941) (end 163.796967 42.035501) (width 0.25) (layer "B.Cu") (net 11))
 (segment (start 163.796967 42.035501) (end 163.796967 42.42441) (width 0.25) (layer "B.Cu") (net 11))
 (segment (start 155.541967 35.38441) (end 155.541967 36.33441) (width 0.25) (layer "B.Cu") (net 11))
 (via (at 147.286967 32.26441) (size 0.8) (drill 0.4) (layers "F.Cu" "B.Cu") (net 14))
 (segment (start 153.541967 34.298014) (end 153.203363 33.95941) (width 0.25) (layer "B.Cu") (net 14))
 (segment (start 148.981967 33.95941) (end 147.286967 32.26441) (width 0.25) (layer "B.Cu") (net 14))
 (segment (start 153.541967 35.38441) (end 153.541967 34.298014) (width 0.25) (layer "B.Cu") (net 14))
 (segment (start 153.203363 33.95941) (end 148.981967 33.95941) (width 0.25) (layer "B.Cu") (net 14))
 (via (at 147.286967 34.80441) (size 0.8) (drill 0.4) (layers "F.Cu" "B.Cu") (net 15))
 (segment (start 147.681967 34.40941) (end 147.286967 34.80441) (width 0.25) (layer "B.Cu") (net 15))
 (segment (start 153.041967 34.43441) (end 153.016967 34.40941) (width 0.25) (layer "B.Cu") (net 15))
 (segment (start 153.016967 34.40941) (end 147.681967 34.40941) (width 0.25) (layer "B.Cu") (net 15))
 (segment (start 153.041967 35.38441) (end 153.041967 34.43441) (width 0.25) (layer "B.Cu") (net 15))
 (via (at 147.286967 37.34441) (size 0.8) (drill 0.4) (layers "F.Cu" "B.Cu") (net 16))
 (segment (start 149.08059 34.85941) (end 147.286967 36.653033) (width 0.25) (layer "B.Cu") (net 16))
 (segment (start 152.541967 35.38441) (end 152.016967 34.85941) (width 0.25) (layer "B.Cu") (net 16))
 (segment (start 147.286967 36.653033) (end 147.286967 37.34441) (width 0.25) (layer "B.Cu") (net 16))
 (segment (start 152.016967 34.85941) (end 149.08059 34.85941) (width 0.25) (layer "B.Cu") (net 16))
 (segment (start 147.433967 44.81741) (end 160.52741 44.81741) (width 0.4) (layer "F.Cu") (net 1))
 (segment (start 147.286967 44.96441) (end 147.433967 44.81741) (width 0.4) (layer "F.Cu") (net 1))
 (segment (start 148.211967 44.96441) (end 149.441967 43.73441) (width 0.4) (layer "F.Cu") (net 1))
 (segment (start 167.247557 46.24) (end 167.291967 46.28441) (width 0.4) (layer "F.Cu") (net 1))
 (segment (start 147.286967 44.96441) (end 148.211967 44.96441) (width 0.4) (layer "F.Cu") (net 1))
 (segment (start 161.95 46.24) (end 167.247557 46.24) (width 0.4) (layer "F.Cu") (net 1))
 (segment (start 160.52741 44.81741) (end 161.95 46.24) (width 0.4) (layer "F.Cu") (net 1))
 (via (at 149.441967 43.73441) (size 0.8) (drill 0.4) (layers "F.Cu" "B.Cu") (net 1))
 (segment (start 154.271967 45.10441) (end 154.271967 45.91741) (width 0.25) (layer "B.Cu") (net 1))
 (segment (start 155.641967 43.73441) (end 149.441967 43.73441) (width 0.25) (layer "B.Cu") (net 1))
 (segment (start 155.641967 43.73441) (end 154.271967 45.10441) (width 0.25) (layer "B.Cu") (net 1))
 (segment (start 160.83 40.655534) (end 160.350876 40.17641) (width 0.4) (layer "B.Cu") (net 8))
 (segment (start 160.83 45.55) (end 160.83 40.655534) (width 0.4) (layer "B.Cu") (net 8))
 (segment (start 145.541967 46.661967) (end 148.04 49.16) (width 0.4) (layer "B.Cu") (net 8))
 (segment (start 148.04 49.16) (end 157.22 49.16) (width 0.4) (layer "B.Cu") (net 8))
 (segment (start 157.22 49.16) (end 160.83 45.55) (width 0.4) (layer "B.Cu") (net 8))
 (segment (start 145.541967 45.61941) (end 145.541967 46.661967) (width 0.4) (layer "B.Cu") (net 8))
 (segment (start 156.866967 45.86241) (end 156.811967 45.91741) (width 0.25) (layer "B.Cu") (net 2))
 (segment (start 155.641967 40.03441) (end 149.441967 40.03441) (width 0.25) (layer "B.Cu") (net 2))
 (segment (start 155.641967 40.03441) (end 156.866967 41.25941) (width 0.25) (layer "B.Cu") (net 2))
 (segment (start 156.866967 41.25941) (end 156.866967 45.86241) (width 0.25) (layer "B.Cu") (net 2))
 (segment (start 147.782557 49.76) (end 165.816377 49.76) (width 0.4) (layer "B.Cu") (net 5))
 (segment (start 165.816377 49.76) (end 167.291967 48.28441) (width 0.4) (layer "B.Cu") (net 5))
 (segment (start 144.041967 45.61941) (end 144.041967 46.01941) (width 0.4) (layer "B.Cu") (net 5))
 (segment (start 144.041967 46.01941) (end 147.782557 49.76) (width 0.4) (layer "B.Cu") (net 5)))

